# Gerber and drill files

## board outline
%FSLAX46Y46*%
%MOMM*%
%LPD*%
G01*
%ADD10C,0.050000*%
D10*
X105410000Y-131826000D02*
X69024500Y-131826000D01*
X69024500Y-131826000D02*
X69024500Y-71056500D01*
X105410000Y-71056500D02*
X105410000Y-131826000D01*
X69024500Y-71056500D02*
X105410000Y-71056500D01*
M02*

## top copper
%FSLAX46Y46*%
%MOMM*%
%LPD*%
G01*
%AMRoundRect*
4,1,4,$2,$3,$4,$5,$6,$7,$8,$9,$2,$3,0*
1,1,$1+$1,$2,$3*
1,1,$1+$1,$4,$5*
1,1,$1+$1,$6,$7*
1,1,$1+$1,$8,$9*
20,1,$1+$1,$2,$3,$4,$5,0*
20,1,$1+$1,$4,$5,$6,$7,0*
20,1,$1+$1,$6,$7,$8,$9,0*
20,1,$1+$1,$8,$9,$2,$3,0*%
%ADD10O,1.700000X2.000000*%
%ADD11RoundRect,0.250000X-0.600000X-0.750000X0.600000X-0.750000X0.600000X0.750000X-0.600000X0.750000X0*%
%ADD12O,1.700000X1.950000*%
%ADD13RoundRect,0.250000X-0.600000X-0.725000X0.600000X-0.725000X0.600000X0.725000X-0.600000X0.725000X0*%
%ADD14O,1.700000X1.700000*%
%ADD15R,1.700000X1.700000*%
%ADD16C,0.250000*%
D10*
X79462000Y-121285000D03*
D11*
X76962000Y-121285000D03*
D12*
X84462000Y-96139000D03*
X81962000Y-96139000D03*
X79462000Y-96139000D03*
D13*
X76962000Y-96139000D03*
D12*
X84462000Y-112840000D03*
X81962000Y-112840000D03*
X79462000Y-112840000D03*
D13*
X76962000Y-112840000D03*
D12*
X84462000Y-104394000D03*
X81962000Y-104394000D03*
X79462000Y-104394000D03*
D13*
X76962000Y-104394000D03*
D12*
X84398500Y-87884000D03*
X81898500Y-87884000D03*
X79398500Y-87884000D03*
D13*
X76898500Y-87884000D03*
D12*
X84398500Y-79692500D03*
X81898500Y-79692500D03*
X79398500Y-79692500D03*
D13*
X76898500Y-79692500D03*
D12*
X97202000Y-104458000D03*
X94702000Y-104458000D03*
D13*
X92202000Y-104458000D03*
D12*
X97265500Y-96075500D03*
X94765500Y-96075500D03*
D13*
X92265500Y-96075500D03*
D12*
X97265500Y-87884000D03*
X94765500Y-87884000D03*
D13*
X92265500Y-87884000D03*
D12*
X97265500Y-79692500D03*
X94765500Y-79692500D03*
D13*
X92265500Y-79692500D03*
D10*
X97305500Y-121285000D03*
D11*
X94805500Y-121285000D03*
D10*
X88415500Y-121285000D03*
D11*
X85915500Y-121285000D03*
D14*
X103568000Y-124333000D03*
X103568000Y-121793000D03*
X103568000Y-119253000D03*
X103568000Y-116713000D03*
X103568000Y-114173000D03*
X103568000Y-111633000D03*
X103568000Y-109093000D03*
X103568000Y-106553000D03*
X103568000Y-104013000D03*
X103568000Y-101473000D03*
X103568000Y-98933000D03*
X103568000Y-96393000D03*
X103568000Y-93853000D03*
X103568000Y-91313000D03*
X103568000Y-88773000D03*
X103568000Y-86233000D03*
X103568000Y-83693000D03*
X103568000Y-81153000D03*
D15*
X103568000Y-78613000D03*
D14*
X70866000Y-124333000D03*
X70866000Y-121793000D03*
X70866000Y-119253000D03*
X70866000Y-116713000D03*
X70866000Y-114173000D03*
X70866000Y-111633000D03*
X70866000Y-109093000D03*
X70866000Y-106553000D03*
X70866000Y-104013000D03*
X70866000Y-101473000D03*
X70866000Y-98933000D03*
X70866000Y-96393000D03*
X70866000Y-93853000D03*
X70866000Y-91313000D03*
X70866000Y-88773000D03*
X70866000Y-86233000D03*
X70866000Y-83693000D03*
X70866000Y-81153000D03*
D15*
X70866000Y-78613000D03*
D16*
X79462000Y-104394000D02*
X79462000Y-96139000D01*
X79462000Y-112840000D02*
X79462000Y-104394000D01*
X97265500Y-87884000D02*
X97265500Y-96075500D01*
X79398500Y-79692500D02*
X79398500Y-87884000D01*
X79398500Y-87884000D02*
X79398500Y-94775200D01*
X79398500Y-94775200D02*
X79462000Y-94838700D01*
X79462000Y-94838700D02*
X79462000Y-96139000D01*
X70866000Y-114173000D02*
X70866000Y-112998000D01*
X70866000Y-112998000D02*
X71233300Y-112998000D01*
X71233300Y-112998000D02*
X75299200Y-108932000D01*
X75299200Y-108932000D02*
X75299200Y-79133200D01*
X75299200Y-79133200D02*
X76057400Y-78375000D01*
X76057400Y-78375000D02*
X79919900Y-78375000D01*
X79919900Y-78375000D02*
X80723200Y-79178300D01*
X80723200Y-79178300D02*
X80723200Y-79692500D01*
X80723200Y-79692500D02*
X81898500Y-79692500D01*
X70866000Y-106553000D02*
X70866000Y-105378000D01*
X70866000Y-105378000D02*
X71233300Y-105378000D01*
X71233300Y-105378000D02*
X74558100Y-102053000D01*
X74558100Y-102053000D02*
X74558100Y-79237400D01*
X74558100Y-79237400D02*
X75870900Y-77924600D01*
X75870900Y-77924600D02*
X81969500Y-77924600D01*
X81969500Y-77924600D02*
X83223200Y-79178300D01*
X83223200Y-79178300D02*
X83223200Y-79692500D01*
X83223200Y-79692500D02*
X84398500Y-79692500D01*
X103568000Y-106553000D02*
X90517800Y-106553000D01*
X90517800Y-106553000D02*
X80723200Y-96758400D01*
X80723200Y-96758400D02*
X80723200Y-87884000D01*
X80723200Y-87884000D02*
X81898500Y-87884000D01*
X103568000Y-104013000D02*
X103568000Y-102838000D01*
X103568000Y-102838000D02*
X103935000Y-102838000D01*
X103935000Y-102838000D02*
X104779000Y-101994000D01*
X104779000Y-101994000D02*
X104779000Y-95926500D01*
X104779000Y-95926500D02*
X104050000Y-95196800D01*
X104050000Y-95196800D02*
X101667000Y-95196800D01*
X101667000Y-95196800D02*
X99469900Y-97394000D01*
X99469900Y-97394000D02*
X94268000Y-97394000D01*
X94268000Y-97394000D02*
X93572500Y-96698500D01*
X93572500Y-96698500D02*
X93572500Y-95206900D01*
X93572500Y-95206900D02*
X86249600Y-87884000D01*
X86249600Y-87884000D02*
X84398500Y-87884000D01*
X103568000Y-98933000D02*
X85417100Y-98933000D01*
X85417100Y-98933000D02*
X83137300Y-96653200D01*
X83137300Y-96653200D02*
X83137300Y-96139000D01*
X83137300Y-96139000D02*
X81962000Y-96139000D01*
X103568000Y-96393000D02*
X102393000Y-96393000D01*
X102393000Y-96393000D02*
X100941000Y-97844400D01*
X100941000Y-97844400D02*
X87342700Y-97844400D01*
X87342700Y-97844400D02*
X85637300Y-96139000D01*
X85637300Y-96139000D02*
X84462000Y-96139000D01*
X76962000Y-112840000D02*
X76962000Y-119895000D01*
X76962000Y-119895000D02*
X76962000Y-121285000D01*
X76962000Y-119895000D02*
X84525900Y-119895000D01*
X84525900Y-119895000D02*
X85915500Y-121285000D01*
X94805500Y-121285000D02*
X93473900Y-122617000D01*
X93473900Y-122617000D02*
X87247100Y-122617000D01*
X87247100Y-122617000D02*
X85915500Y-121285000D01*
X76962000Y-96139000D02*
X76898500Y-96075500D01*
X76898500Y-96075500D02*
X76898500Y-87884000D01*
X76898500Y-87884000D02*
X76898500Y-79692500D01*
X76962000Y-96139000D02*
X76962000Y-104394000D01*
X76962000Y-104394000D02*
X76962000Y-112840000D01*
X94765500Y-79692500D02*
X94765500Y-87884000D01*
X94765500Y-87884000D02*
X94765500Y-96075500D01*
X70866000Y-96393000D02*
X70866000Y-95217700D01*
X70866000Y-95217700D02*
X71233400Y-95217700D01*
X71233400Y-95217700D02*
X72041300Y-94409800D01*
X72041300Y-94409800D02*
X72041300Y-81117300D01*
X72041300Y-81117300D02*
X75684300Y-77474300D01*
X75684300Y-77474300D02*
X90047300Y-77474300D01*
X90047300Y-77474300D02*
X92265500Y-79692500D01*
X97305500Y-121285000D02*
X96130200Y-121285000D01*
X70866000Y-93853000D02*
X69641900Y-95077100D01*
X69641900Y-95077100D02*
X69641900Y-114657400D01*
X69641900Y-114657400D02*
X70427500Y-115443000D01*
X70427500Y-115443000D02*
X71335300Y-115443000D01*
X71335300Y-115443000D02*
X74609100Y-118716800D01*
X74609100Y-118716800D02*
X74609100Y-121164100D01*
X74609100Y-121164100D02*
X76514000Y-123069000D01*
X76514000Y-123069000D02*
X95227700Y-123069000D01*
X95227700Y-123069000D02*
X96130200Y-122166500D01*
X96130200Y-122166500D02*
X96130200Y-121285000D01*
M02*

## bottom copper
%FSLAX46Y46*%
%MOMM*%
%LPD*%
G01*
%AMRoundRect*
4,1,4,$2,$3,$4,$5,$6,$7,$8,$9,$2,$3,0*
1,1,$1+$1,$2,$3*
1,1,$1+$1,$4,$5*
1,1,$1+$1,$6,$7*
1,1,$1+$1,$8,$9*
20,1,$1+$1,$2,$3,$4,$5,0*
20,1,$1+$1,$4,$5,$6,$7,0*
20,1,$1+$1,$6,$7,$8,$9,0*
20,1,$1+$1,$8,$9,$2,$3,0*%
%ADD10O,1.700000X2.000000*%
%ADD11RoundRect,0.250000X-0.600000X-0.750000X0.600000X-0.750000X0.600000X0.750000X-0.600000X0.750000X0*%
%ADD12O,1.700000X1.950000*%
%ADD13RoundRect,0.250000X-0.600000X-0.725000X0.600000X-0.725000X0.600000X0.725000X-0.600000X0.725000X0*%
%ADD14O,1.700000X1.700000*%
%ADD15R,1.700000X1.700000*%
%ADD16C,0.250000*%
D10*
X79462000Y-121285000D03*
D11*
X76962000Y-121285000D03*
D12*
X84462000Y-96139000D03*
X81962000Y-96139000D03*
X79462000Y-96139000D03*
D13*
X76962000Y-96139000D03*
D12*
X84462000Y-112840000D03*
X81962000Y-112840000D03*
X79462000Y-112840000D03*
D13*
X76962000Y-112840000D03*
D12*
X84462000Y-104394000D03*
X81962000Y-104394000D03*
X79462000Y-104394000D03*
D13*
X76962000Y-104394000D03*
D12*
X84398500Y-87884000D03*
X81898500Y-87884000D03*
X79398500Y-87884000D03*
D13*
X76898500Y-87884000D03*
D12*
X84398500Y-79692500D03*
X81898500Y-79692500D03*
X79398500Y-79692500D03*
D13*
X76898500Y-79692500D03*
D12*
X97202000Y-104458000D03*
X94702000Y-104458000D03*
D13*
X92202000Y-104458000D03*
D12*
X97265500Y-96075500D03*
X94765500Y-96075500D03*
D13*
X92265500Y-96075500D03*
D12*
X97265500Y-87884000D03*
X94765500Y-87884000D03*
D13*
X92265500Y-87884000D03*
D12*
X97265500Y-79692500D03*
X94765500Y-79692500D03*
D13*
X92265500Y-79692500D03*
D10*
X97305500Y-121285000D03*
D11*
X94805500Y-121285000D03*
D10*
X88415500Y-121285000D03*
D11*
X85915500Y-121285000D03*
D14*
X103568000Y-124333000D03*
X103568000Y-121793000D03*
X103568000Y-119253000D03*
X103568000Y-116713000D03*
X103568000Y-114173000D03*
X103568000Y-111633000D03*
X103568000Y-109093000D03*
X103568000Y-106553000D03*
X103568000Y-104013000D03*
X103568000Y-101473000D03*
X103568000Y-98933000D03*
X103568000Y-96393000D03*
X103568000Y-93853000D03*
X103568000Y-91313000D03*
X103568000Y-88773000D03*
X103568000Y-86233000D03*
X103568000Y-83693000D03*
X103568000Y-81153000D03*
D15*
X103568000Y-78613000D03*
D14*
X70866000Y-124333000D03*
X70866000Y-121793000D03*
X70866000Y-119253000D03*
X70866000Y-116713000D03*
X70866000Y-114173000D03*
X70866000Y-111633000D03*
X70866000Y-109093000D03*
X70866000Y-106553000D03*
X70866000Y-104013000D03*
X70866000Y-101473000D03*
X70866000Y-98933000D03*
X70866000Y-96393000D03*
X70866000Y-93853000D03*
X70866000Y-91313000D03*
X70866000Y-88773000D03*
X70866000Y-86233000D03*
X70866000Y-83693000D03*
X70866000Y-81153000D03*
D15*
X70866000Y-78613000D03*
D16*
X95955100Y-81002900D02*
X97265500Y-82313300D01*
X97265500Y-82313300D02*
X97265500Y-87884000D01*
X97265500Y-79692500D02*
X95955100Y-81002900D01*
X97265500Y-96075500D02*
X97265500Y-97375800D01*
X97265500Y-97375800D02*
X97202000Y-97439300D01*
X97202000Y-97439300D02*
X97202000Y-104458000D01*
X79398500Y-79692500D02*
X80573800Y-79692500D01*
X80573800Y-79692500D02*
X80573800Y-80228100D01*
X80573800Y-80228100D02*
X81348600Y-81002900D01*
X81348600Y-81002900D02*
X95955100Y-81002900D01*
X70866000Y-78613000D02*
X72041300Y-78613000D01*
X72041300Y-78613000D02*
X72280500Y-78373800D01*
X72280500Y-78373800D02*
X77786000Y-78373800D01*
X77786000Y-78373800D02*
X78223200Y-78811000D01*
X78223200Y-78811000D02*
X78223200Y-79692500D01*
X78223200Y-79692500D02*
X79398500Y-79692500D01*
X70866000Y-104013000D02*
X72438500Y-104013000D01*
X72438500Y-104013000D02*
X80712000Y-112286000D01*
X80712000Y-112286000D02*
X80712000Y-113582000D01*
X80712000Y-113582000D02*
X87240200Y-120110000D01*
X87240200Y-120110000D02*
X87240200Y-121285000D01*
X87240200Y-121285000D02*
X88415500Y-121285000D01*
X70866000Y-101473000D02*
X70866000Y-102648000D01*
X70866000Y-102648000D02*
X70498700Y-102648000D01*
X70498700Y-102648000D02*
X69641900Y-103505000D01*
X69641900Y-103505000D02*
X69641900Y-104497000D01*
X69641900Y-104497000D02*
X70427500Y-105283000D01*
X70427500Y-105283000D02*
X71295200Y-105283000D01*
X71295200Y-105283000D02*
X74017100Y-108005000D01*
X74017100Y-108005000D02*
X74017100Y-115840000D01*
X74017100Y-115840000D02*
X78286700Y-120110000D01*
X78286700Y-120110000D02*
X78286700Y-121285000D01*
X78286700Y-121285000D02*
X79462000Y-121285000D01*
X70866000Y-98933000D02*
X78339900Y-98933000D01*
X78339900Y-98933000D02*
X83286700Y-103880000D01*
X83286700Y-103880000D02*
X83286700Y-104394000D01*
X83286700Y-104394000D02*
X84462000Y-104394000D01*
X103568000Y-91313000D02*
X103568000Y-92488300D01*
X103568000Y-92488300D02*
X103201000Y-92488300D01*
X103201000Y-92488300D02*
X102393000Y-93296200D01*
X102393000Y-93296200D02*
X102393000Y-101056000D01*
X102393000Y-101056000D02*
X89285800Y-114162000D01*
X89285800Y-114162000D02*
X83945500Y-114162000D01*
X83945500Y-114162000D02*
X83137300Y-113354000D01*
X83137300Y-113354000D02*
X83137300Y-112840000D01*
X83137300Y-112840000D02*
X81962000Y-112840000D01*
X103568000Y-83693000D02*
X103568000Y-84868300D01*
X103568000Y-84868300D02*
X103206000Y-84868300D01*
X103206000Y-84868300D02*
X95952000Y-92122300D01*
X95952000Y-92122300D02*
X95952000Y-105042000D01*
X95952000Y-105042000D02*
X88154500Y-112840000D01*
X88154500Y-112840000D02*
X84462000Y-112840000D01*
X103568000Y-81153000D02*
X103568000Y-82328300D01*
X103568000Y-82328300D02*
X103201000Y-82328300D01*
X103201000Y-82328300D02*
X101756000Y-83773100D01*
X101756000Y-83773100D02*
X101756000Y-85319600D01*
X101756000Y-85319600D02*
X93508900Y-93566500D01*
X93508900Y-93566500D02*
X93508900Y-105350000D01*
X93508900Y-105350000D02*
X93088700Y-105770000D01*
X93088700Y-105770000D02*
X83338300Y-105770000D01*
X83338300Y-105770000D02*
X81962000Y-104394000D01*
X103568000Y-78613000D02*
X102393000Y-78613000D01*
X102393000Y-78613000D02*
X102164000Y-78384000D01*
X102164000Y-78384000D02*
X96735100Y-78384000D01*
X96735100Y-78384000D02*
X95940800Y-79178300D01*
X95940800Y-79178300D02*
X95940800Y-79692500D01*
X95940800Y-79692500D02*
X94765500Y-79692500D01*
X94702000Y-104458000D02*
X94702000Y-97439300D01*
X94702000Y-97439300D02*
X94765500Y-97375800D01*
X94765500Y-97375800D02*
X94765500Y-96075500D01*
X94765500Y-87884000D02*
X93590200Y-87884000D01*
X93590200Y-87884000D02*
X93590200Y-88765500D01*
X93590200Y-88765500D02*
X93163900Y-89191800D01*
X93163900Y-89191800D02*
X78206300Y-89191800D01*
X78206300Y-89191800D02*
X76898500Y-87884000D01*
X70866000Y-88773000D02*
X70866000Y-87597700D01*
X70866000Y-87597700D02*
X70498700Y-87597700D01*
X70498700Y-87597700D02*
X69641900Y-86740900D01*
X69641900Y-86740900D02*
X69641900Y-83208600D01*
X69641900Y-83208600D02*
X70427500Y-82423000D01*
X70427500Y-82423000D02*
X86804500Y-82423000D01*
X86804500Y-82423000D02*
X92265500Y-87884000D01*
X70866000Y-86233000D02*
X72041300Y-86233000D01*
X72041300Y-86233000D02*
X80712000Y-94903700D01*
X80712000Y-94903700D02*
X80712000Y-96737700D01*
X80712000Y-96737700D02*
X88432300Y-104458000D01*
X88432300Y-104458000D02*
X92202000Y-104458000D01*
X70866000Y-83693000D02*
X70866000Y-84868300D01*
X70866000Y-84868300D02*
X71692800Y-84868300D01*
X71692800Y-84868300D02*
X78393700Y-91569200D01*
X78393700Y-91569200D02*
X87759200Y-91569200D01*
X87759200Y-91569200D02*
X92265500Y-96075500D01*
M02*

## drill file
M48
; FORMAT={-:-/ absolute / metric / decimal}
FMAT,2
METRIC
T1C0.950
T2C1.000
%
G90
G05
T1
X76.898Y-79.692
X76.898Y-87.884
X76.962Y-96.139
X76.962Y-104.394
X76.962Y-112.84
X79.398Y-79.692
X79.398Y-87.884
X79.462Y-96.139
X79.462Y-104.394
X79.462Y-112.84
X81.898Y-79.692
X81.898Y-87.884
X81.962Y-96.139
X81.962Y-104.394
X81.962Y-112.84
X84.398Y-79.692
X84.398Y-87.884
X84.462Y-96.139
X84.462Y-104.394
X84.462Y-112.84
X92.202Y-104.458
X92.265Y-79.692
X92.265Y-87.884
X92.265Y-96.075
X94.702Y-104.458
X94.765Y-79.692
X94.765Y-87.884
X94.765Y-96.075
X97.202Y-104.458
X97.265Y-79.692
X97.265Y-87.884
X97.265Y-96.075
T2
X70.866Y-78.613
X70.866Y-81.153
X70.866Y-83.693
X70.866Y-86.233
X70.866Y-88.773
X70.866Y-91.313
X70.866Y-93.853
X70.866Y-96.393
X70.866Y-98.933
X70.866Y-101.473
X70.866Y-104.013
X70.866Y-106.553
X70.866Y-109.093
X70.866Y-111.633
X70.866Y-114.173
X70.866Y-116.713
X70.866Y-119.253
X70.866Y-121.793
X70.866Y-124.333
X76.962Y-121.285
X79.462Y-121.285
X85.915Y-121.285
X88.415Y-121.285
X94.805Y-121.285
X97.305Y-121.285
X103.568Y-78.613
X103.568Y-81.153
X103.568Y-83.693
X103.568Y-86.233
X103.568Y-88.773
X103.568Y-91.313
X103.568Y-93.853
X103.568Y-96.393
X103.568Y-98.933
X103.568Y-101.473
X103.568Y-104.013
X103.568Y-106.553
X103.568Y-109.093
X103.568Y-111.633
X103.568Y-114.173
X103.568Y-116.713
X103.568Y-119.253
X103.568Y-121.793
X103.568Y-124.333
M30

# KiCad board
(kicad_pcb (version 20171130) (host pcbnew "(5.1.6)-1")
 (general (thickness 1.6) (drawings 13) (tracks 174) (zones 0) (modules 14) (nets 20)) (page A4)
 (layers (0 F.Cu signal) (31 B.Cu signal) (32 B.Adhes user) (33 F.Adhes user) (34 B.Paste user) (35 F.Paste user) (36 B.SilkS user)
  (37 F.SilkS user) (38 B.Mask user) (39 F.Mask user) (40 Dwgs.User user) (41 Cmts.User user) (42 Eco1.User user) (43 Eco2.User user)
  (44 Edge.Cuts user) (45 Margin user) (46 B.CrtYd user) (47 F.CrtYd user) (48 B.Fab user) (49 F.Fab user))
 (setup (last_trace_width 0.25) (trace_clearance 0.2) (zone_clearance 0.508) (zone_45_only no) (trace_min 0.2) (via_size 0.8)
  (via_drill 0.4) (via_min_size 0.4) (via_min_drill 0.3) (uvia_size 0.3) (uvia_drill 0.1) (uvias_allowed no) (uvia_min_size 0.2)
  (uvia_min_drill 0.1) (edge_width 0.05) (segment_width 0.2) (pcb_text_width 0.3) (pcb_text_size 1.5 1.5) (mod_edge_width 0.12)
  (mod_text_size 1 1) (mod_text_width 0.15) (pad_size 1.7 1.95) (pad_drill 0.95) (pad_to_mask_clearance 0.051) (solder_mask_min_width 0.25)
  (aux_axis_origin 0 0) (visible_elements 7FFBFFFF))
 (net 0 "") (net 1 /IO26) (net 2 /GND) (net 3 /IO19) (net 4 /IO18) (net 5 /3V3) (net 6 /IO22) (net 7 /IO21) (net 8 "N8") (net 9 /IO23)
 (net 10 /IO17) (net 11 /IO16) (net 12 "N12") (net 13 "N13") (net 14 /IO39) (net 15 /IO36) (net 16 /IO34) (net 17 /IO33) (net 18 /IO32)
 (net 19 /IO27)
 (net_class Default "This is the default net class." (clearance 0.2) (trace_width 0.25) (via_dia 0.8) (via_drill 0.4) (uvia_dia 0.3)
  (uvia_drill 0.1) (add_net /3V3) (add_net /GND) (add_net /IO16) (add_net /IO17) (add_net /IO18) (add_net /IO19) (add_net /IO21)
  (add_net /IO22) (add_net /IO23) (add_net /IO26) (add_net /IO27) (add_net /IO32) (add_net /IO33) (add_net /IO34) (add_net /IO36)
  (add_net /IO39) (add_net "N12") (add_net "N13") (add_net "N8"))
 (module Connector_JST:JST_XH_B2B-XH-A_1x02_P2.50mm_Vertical (layer F.Cu) (at 76.962 121.285)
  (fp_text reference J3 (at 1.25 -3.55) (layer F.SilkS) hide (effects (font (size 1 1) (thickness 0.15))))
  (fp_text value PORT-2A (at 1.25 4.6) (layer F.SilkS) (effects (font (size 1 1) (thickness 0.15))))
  (pad 2 thru_hole oval (at 2.5 0) (size 1.7 2) (drill 1) (layers *.Cu *.Mask) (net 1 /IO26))
  (pad 1 thru_hole roundrect (at 0 0) (size 1.7 2) (drill 1) (layers *.Cu *.Mask) (roundrect_rratio 0.147059) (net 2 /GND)))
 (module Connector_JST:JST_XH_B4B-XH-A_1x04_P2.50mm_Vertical (layer F.Cu) (at 76.962 96.139)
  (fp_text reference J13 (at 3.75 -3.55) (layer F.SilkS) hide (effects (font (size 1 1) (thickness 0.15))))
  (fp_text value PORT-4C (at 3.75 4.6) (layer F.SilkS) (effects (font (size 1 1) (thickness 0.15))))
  (pad 4 thru_hole oval (at 7.5 0) (size 1.7 1.95) (drill 0.95) (layers *.Cu *.Mask) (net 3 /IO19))
  (pad 3 thru_hole oval (at 5 0) (size 1.7 1.95) (drill 0.95) (layers *.Cu *.Mask) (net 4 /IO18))
  (pad 2 thru_hole oval (at 2.5 0) (size 1.7 1.95) (drill 0.95) (layers *.Cu *.Mask) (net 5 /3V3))
  (pad 1 thru_hole roundrect (at 0 0) (size 1.7 1.95) (drill 0.95) (layers *.Cu *.Mask) (roundrect_rratio 0.147059) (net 2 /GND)))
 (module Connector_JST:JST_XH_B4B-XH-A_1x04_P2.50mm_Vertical (layer F.Cu) (at 76.962 112.84)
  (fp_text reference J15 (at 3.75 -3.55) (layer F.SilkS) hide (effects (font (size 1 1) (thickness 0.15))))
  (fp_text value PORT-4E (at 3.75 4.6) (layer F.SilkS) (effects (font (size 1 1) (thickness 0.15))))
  (pad 4 thru_hole oval (at 7.5 0) (size 1.7 1.95) (drill 0.95) (layers *.Cu *.Mask) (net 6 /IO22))
  (pad 3 thru_hole oval (at 5 0) (size 1.7 1.95) (drill 0.95) (layers *.Cu *.Mask) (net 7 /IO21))
  (pad 2 thru_hole oval (at 2.5 0) (size 1.7 1.95) (drill 0.95) (layers *.Cu *.Mask) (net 5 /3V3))
  (pad 1 thru_hole roundrect (at 0 0) (size 1.7 1.95) (drill 0.95) (layers *.Cu *.Mask) (roundrect_rratio 0.147059) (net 2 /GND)))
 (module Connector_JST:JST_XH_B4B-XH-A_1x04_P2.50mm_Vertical (layer F.Cu) (at 76.962 104.394)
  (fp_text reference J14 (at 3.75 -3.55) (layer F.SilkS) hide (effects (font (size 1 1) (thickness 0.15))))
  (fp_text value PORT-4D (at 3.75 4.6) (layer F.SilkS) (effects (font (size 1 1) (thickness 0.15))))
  (pad 4 thru_hole oval (at 7.5 0) (size 1.7 1.95) (drill 0.95) (layers *.Cu *.Mask) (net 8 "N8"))
  (pad 3 thru_hole oval (at 5 0) (size 1.7 1.95) (drill 0.95) (layers *.Cu *.Mask) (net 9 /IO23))
  (pad 2 thru_hole oval (at 2.5 0) (size 1.7 1.95) (drill 0.95) (layers *.Cu *.Mask) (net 5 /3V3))
  (pad 1 thru_hole roundrect (at 0 0) (size 1.7 1.95) (drill 0.95) (layers *.Cu *.Mask) (roundrect_rratio 0.147059) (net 2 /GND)))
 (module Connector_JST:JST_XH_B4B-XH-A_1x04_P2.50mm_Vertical (layer F.Cu) (at 76.8985 87.884)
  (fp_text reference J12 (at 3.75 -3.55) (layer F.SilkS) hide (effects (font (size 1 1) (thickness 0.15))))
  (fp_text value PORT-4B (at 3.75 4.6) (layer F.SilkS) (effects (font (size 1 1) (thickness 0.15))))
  (pad 4 thru_hole oval (at 7.5 0) (size 1.7 1.95) (drill 0.95) (layers *.Cu *.Mask) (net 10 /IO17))
  (pad 3 thru_hole oval (at 5 0) (size 1.7 1.95) (drill 0.95) (layers *.Cu *.Mask) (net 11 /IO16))
  (pad 2 thru_hole oval (at 2.5 0) (size 1.7 1.95) (drill 0.95) (layers *.Cu *.Mask) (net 5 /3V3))
  (pad 1 thru_hole roundrect (at 0 0) (size 1.7 1.95) (drill 0.95) (layers *.Cu *.Mask) (roundrect_rratio 0.147059) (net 2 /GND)))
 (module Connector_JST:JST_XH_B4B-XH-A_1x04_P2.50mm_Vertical (layer F.Cu) (at 76.8985 79.6925)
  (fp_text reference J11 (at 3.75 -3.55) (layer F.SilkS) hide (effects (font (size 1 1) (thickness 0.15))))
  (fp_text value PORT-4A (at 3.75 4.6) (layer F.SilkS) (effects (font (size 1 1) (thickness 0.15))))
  (pad 4 thru_hole oval (at 7.5 0) (size 1.7 1.95) (drill 0.95) (layers *.Cu *.Mask) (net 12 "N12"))
  (pad 3 thru_hole oval (at 5 0) (size 1.7 1.95) (drill 0.95) (layers *.Cu *.Mask) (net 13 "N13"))
  (pad 2 thru_hole oval (at 2.5 0) (size 1.7 1.95) (drill 0.95) (layers *.Cu *.Mask) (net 5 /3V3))
  (pad 1 thru_hole roundrect (at 0 0) (size 1.7 1.95) (drill 0.95) (layers *.Cu *.Mask) (roundrect_rratio 0.147059) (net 2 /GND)))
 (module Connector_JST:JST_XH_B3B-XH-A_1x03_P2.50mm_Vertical (layer F.Cu) (at 92.202 104.458)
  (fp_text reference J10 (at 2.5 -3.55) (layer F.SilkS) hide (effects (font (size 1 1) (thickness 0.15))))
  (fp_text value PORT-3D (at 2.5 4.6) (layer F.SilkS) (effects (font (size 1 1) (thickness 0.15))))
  (pad 3 thru_hole oval (at 5 0) (size 1.7 1.95) (drill 0.95) (layers *.Cu *.Mask) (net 5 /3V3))
  (pad 2 thru_hole oval (at 2.5 0) (size 1.7 1.95) (drill 0.95) (layers *.Cu *.Mask) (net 2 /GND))
  (pad 1 thru_hole roundrect (at 0 0) (size 1.7 1.95) (drill 0.95) (layers *.Cu *.Mask) (roundrect_rratio 0.147059) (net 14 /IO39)))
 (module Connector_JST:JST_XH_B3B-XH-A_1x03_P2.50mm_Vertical (layer F.Cu) (at 92.2655 96.0755)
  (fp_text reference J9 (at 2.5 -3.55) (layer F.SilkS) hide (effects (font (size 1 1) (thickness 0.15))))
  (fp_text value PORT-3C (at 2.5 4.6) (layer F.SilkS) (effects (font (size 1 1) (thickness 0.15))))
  (pad 3 thru_hole oval (at 5 0) (size 1.7 1.95) (drill 0.95) (layers *.Cu *.Mask) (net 5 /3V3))
  (pad 2 thru_hole oval (at 2.5 0) (size 1.7 1.95) (drill 0.95) (layers *.Cu *.Mask) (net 2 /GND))
  (pad 1 thru_hole roundrect (at 0 0) (size 1.7 1.95) (drill 0.95) (layers *.Cu *.Mask) (roundrect_rratio 0.147059) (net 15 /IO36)))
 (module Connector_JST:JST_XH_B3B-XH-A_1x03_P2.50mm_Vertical (layer F.Cu) (at 92.2655 87.884)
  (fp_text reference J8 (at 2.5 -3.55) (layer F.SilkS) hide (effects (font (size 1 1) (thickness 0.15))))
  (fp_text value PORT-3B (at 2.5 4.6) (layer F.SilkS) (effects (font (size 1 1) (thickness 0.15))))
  (pad 3 thru_hole oval (at 5 0) (size 1.7 1.95) (drill 0.95) (layers *.Cu *.Mask) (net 5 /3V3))
  (pad 2 thru_hole oval (at 2.5 0) (size 1.7 1.95) (drill 0.95) (layers *.Cu *.Mask) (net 2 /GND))
  (pad 1 thru_hole roundrect (at 0 0) (size 1.7 1.95) (drill 0.95) (layers *.Cu *.Mask) (roundrect_rratio 0.147059) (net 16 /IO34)))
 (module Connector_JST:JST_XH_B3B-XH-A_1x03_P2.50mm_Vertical (layer F.Cu) (at 92.2655 79.6925)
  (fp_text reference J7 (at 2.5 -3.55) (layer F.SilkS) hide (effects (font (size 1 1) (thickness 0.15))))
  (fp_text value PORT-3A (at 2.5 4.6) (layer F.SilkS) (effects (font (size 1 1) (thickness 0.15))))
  (pad 3 thru_hole oval (at 5 0) (size 1.7 1.95) (drill 0.95) (layers *.Cu *.Mask) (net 5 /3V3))
  (pad 2 thru_hole oval (at 2.5 0) (size 1.7 1.95) (drill 0.95) (layers *.Cu *.Mask) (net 2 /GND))
  (pad 1 thru_hole roundrect (at 0 0) (size 1.7 1.95) (drill 0.95) (layers *.Cu *.Mask) (roundrect_rratio 0.147059) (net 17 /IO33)))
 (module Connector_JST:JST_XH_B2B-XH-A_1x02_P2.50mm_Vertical (layer F.Cu) (at 94.8055 121.285)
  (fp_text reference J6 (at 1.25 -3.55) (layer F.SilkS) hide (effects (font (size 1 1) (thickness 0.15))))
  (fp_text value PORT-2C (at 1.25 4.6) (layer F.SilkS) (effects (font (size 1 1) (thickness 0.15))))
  (pad 2 thru_hole oval (at 2.5 0) (size 1.7 2) (drill 1) (layers *.Cu *.Mask) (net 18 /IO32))
  (pad 1 thru_hole roundrect (at 0 0) (size 1.7 2) (drill 1) (layers *.Cu *.Mask) (roundrect_rratio 0.147059) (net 2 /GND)))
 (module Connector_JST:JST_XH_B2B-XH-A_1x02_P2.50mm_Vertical (layer F.Cu) (at 85.9155 121.285)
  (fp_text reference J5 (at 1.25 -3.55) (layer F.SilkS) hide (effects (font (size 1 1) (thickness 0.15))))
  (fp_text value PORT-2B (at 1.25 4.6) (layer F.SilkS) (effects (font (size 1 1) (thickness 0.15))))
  (pad 2 thru_hole oval (at 2.5 0) (size 1.7 2) (drill 1) (layers *.Cu *.Mask) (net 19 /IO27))
  (pad 1 thru_hole roundrect (at 0 0) (size 1.7 2) (drill 1) (layers *.Cu *.Mask) (roundrect_rratio 0.147059) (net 2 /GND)))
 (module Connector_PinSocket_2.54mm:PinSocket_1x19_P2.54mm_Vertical (layer F.Cu) (at 103.568 78.613)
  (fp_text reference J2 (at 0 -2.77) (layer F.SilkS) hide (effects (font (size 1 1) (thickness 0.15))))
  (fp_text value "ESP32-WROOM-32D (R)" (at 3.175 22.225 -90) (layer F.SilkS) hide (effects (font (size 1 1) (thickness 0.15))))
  (pad 19 thru_hole oval (at 0 45.72) (size 1.7 1.7) (drill 1) (layers *.Cu *.Mask))
  (pad 18 thru_hole oval (at 0 43.18) (size 1.7 1.7) (drill 1) (layers *.Cu *.Mask))
  (pad 17 thru_hole oval (at 0 40.64) (size 1.7 1.7) (drill 1) (layers *.Cu *.Mask))
  (pad 16 thru_hole oval (at 0 38.1) (size 1.7 1.7) (drill 1) (layers *.Cu *.Mask))
  (pad 15 thru_hole oval (at 0 35.56) (size 1.7 1.7) (drill 1) (layers *.Cu *.Mask))
  (pad 14 thru_hole oval (at 0 33.02) (size 1.7 1.7) (drill 1) (layers *.Cu *.Mask))
  (pad 13 thru_hole oval (at 0 30.48) (size 1.7 1.7) (drill 1) (layers *.Cu *.Mask))
  (pad 12 thru_hole oval (at 0 27.94) (size 1.7 1.7) (drill 1) (layers *.Cu *.Mask) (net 11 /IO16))
  (pad 11 thru_hole oval (at 0 25.4) (size 1.7 1.7) (drill 1) (layers *.Cu *.Mask) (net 10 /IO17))
  (pad 10 thru_hole oval (at 0 22.86) (size 1.7 1.7) (drill 1) (layers *.Cu *.Mask))
  (pad 9 thru_hole oval (at 0 20.32) (size 1.7 1.7) (drill 1) (layers *.Cu *.Mask) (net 4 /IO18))
  (pad 8 thru_hole oval (at 0 17.78) (size 1.7 1.7) (drill 1) (layers *.Cu *.Mask) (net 3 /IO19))
  (pad 7 thru_hole oval (at 0 15.24) (size 1.7 1.7) (drill 1) (layers *.Cu *.Mask))
  (pad 6 thru_hole oval (at 0 12.7) (size 1.7 1.7) (drill 1) (layers *.Cu *.Mask) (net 7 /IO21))
  (pad 5 thru_hole oval (at 0 10.16) (size 1.7 1.7) (drill 1) (layers *.Cu *.Mask))
  (pad 4 thru_hole oval (at 0 7.62) (size 1.7 1.7) (drill 1) (layers *.Cu *.Mask))
  (pad 3 thru_hole oval (at 0 5.08) (size 1.7 1.7) (drill 1) (layers *.Cu *.Mask) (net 6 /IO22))
  (pad 2 thru_hole oval (at 0 2.54) (size 1.7 1.7) (drill 1) (layers *.Cu *.Mask) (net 9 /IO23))
  (pad 1 thru_hole rect (at 0 0) (size 1.7 1.7) (drill 1) (layers *.Cu *.Mask) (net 2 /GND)))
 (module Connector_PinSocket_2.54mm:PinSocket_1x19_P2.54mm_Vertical (layer F.Cu) (at 70.866 78.613)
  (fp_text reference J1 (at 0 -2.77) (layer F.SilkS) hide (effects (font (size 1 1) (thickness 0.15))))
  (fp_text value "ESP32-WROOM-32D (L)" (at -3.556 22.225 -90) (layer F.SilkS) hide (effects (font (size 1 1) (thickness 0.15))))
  (pad 19 thru_hole oval (at 0 45.72) (size 1.7 1.7) (drill 1) (layers *.Cu *.Mask))
  (pad 18 thru_hole oval (at 0 43.18) (size 1.7 1.7) (drill 1) (layers *.Cu *.Mask))
  (pad 17 thru_hole oval (at 0 40.64) (size 1.7 1.7) (drill 1) (layers *.Cu *.Mask))
  (pad 16 thru_hole oval (at 0 38.1) (size 1.7 1.7) (drill 1) (layers *.Cu *.Mask))
  (pad 15 thru_hole oval (at 0 35.56) (size 1.7 1.7) (drill 1) (layers *.Cu *.Mask) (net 13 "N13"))
  (pad 14 thru_hole oval (at 0 33.02) (size 1.7 1.7) (drill 1) (layers *.Cu *.Mask))
  (pad 13 thru_hole oval (at 0 30.48) (size 1.7 1.7) (drill 1) (layers *.Cu *.Mask))
  (pad 12 thru_hole oval (at 0 27.94) (size 1.7 1.7) (drill 1) (layers *.Cu *.Mask) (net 12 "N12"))
  (pad 11 thru_hole oval (at 0 25.4) (size 1.7 1.7) (drill 1) (layers *.Cu *.Mask) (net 19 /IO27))
  (pad 10 thru_hole oval (at 0 22.86) (size 1.7 1.7) (drill 1) (layers *.Cu *.Mask) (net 1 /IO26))
  (pad 9 thru_hole oval (at 0 20.32) (size 1.7 1.7) (drill 1) (layers *.Cu *.Mask) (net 8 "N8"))
  (pad 8 thru_hole oval (at 0 17.78) (size 1.7 1.7) (drill 1) (layers *.Cu *.Mask) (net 17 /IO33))
  (pad 7 thru_hole oval (at 0 15.24) (size 1.7 1.7) (drill 1) (layers *.Cu *.Mask) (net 18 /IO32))
  (pad 6 thru_hole oval (at 0 12.7) (size 1.7 1.7) (drill 1) (layers *.Cu *.Mask))
  (pad 5 thru_hole oval (at 0 10.16) (size 1.7 1.7) (drill 1) (layers *.Cu *.Mask) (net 16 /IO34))
  (pad 4 thru_hole oval (at 0 7.62) (size 1.7 1.7) (drill 1) (layers *.Cu *.Mask) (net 14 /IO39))
  (pad 3 thru_hole oval (at 0 5.08) (size 1.7 1.7) (drill 1) (layers *.Cu *.Mask) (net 15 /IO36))
  (pad 2 thru_hole oval (at 0 2.54) (size 1.7 1.7) (drill 1) (layers *.Cu *.Mask))
  (pad 1 thru_hole rect (at 0 0) (size 1.7 1.7) (drill 1) (layers *.Cu *.Mask) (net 5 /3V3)))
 (gr_line (start 105.41 131.826) (end 69.0245 131.826) (layer Edge.Cuts) (width 0.05))
 (gr_line (start 69.0245 131.826) (end 69.0245 71.0565) (layer Edge.Cuts) (width 0.05))
 (gr_line (start 105.41 71.0565) (end 105.41 131.826) (layer Edge.Cuts) (width 0.05))
 (gr_line (start 69.0245 71.0565) (end 105.41 71.0565) (layer Edge.Cuts) (width 0.05))
 (segment (start 95.9551 81.0029) (end 97.2655 82.3133) (width 0.25) (layer B.Cu) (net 5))
 (segment (start 97.2655 82.3133) (end 97.2655 87.884) (width 0.25) (layer B.Cu) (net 5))
 (segment (start 97.2655 79.6925) (end 95.9551 81.0029) (width 0.25) (layer B.Cu) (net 5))
 (segment (start 79.462 104.394) (end 79.462 96.139) (width 0.25) (layer F.Cu) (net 5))
 (segment (start 79.462 112.84) (end 79.462 104.394) (width 0.25) (layer F.Cu) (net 5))
 (segment (start 97.2655 87.884) (end 97.2655 96.0755) (width 0.25) (layer F.Cu) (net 5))
 (segment (start 97.2655 96.0755) (end 97.2655 97.3758) (width 0.25) (layer B.Cu) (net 5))
 (segment (start 97.2655 97.3758) (end 97.202 97.4393) (width 0.25) (layer B.Cu) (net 5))
 (segment (start 97.202 97.4393) (end 97.202 104.458) (width 0.25) (layer B.Cu) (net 5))
 (segment (start 79.3985 79.6925) (end 80.5738 79.6925) (width 0.25) (layer B.Cu) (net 5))
 (segment (start 80.5738 79.6925) (end 80.5738 80.2281) (width 0.25) (layer B.Cu) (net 5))
 (segment (start 80.5738 80.2281) (end 81.3486 81.0029) (width 0.25) (layer B.Cu) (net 5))
 (segment (start 81.3486 81.0029) (end 95.9551 81.0029) (width 0.25) (layer B.Cu) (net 5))
 (segment (start 79.3985 79.6925) (end 79.3985 87.884) (width 0.25) (layer F.Cu) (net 5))
 (segment (start 79.3985 87.884) (end 79.3985 94.7752) (width 0.25) (layer F.Cu) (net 5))
 (segment (start 79.3985 94.7752) (end 79.462 94.8387) (width 0.25) (layer F.Cu) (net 5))
 (segment (start 79.462 94.8387) (end 79.462 96.139) (width 0.25) (layer F.Cu) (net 5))
 (segment (start 70.866 78.613) (end 72.0413 78.613) (width 0.25) (layer B.Cu) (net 5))
 (segment (start 72.0413 78.613) (end 72.2805 78.3738) (width 0.25) (layer B.Cu) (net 5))
 (segment (start 72.2805 78.3738) (end 77.786 78.3738) (width 0.25) (layer B.Cu) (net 5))
 (segment (start 77.786 78.3738) (end 78.2232 78.811) (width 0.25) (layer B.Cu) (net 5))
 (segment (start 78.2232 78.811) (end 78.2232 79.6925) (width 0.25) (layer B.Cu) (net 5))
 (segment (start 78.2232 79.6925) (end 79.3985 79.6925) (width 0.25) (layer B.Cu) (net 5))
 (segment (start 70.866 114.173) (end 70.866 112.998) (width 0.25) (layer F.Cu) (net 13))
 (segment (start 70.866 112.998) (end 71.2333 112.998) (width 0.25) (layer F.Cu) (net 13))
 (segment (start 71.2333 112.998) (end 75.2992 108.932) (width 0.25) (layer F.Cu) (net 13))
 (segment (start 75.2992 108.932) (end 75.2992 79.1332) (width 0.25) (layer F.Cu) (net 13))
 (segment (start 75.2992 79.1332) (end 76.0574 78.375) (width 0.25) (layer F.Cu) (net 13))
 (segment (start 76.0574 78.375) (end 79.9199 78.375) (width 0.25) (layer F.Cu) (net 13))
 (segment (start 79.9199 78.375) (end 80.7232 79.1783) (width 0.25) (layer F.Cu) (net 13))
 (segment (start 80.7232 79.1783) (end 80.7232 79.6925) (width 0.25) (layer F.Cu) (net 13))
 (segment (start 80.7232 79.6925) (end 81.8985 79.6925) (width 0.25) (layer F.Cu) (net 13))
 (segment (start 70.866 106.553) (end 70.866 105.378) (width 0.25) (layer F.Cu) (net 12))
 (segment (start 70.866 105.378) (end 71.2333 105.378) (width 0.25) (layer F.Cu) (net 12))
 (segment (start 71.2333 105.378) (end 74.5581 102.053) (width 0.25) (layer F.Cu) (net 12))
 (segment (start 74.5581 102.053) (end 74.5581 79.2374) (width 0.25) (layer F.Cu) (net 12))
 (segment (start 74.5581 79.2374) (end 75.8709 77.9246) (width 0.25) (layer F.Cu) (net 12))
 (segment (start 75.8709 77.9246) (end 81.9695 77.9246) (width 0.25) (layer F.Cu) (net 12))
 (segment (start 81.9695 77.9246) (end 83.2232 79.1783) (width 0.25) (layer F.Cu) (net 12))
 (segment (start 83.2232 79.1783) (end 83.2232 79.6925) (width 0.25) (layer F.Cu) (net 12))
 (segment (start 83.2232 79.6925) (end 84.3985 79.6925) (width 0.25) (layer F.Cu) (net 12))
 (segment (start 70.866 104.013) (end 72.4385 104.013) (width 0.25) (layer B.Cu) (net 19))
 (segment (start 72.4385 104.013) (end 80.712 112.286) (width 0.25) (layer B.Cu) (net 19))
 (segment (start 80.712 112.286) (end 80.712 113.582) (width 0.25) (layer B.Cu) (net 19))
 (segment (start 80.712 113.582) (end 87.2402 120.11) (width 0.25) (layer B.Cu) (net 19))
 (segment (start 87.2402 120.11) (end 87.2402 121.285) (width 0.25) (layer B.Cu) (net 19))
 (segment (start 87.2402 121.285) (end 88.4155 121.285) (width 0.25) (layer B.Cu) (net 19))
 (segment (start 70.866 101.473) (end 70.866 102.648) (width 0.25) (layer B.Cu) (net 1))
 (segment (start 70.866 102.648) (end 70.4987 102.648) (width 0.25) (layer B.Cu) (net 1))
 (segment (start 70.4987 102.648) (end 69.6419 103.505) (width 0.25) (layer B.Cu) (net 1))
 (segment (start 69.6419 103.505) (end 69.6419 104.497) (width 0.25) (layer B.Cu) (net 1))
 (segment (start 69.6419 104.497) (end 70.4275 105.283) (width 0.25) (layer B.Cu) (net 1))
 (segment (start 70.4275 105.283) (end 71.2952 105.283) (width 0.25) (layer B.Cu) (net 1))
 (segment (start 71.2952 105.283) (end 74.0171 108.005) (width 0.25) (layer B.Cu) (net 1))
 (segment (start 74.0171 108.005) (end 74.0171 115.84) (width 0.25) (layer B.Cu) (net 1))
 (segment (start 74.0171 115.84) (end 78.2867 120.11) (width 0.25) (layer B.Cu) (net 1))
 (segment (start 78.2867 120.11) (end 78.2867 121.285) (width 0.25) (layer B.Cu) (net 1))
 (segment (start 78.2867 121.285) (end 79.462 121.285) (width 0.25) (layer B.Cu) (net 1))
 (segment (start 70.866 98.933) (end 78.3399 98.933) (width 0.25) (layer B.Cu) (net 8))
 (segment (start 78.3399 98.933) (end 83.2867 103.88) (width 0.25) (layer B.Cu) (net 8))
 (segment (start 83.2867 103.88) (end 83.2867 104.394) (width 0.25) (layer B.Cu) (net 8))
 (segment (start 83.2867 104.394) (end 84.462 104.394) (width 0.25) (layer B.Cu) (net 8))
 (segment (start 103.568 106.553) (end 90.5178 106.553) (width 0.25) (layer F.Cu) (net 11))
 (segment (start 90.5178 106.553) (end 80.7232 96.7584) (width 0.25) (layer F.Cu) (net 11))
 (segment (start 80.7232 96.7584) (end 80.7232 87.884) (width 0.25) (layer F.Cu) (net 11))
 (segment (start 80.7232 87.884) (end 81.8985 87.884) (width 0.25) (layer F.Cu) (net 11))
 (segment (start 103.568 104.013) (end 103.568 102.838) (width 0.25) (layer F.Cu) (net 10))
 (segment (start 103.568 102.838) (end 103.935 102.838) (width 0.25) (layer F.Cu) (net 10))
 (segment (start 103.935 102.838) (end 104.779 101.994) (width 0.25) (layer F.Cu) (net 10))
 (segment (start 104.779 101.994) (end 104.779 95.9265) (width 0.25) (layer F.Cu) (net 10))
 (segment (start 104.779 95.9265) (end 104.05 95.1968) (width 0.25) (layer F.Cu) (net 10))
 (segment (start 104.05 95.1968) (end 101.667 95.1968) (width 0.25) (layer F.Cu) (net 10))
 (segment (start 101.667 95.1968) (end 99.4699 97.394) (width 0.25) (layer F.Cu) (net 10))
 (segment (start 99.4699 97.394) (end 94.268 97.394) (width 0.25) (layer F.Cu) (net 10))
 (segment (start 94.268 97.394) (end 93.5725 96.6985) (width 0.25) (layer F.Cu) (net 10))
 (segment (start 93.5725 96.6985) (end 93.5725 95.2069) (width 0.25) (layer F.Cu) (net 10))
 (segment (start 93.5725 95.2069) (end 86.2496 87.884) (width 0.25) (layer F.Cu) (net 10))
 (segment (start 86.2496 87.884) (end 84.3985 87.884) (width 0.25) (layer F.Cu) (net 10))
 (segment (start 103.568 98.933) (end 85.4171 98.933) (width 0.25) (layer F.Cu) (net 4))
 (segment (start 85.4171 98.933) (end 83.1373 96.6532) (width 0.25) (layer F.Cu) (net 4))
 (segment (start 83.1373 96.6532) (end 83.1373 96.139) (width 0.25) (layer F.Cu) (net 4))
 (segment (start 83.1373 96.139) (end 81.962 96.139) (width 0.25) (layer F.Cu) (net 4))
 (segment (start 103.568 96.393) (end 102.393 96.393) (width 0.25) (layer F.Cu) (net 3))
 (segment (start 102.393 96.393) (end 100.941 97.8444) (width 0.25) (layer F.Cu) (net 3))
 (segment (start 100.941 97.8444) (end 87.3427 97.8444) (width 0.25) (layer F.Cu) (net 3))
 (segment (start 87.3427 97.8444) (end 85.6373 96.139) (width 0.25) (layer F.Cu) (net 3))
 (segment (start 85.6373 96.139) (end 84.462 96.139) (width 0.25) (layer F.Cu) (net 3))
 (segment (start 103.568 91.313) (end 103.568 92.4883) (width 0.25) (layer B.Cu) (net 7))
 (segment (start 103.568 92.4883) (end 103.201 92.4883) (width 0.25) (layer B.Cu) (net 7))
 (segment (start 103.201 92.4883) (end 102.393 93.2962) (width 0.25) (layer B.Cu) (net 7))
 (segment (start 102.393 93.2962) (end 102.393 101.056) (width 0.25) (layer B.Cu) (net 7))
 (segment (start 102.393 101.056) (end 89.2858 114.162) (width 0.25) (layer B.Cu) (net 7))
 (segment (start 89.2858 114.162) (end 83.9455 114.162) (width 0.25) (layer B.Cu) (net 7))
 (segment (start 83.9455 114.162) (end 83.1373 113.354) (width 0.25) (layer B.Cu) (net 7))
 (segment (start 83.1373 113.354) (end 83.1373 112.84) (width 0.25) (layer B.Cu) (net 7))
 (segment (start 83.1373 112.84) (end 81.962 112.84) (width 0.25) (layer B.Cu) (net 7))
 (segment (start 103.568 83.693) (end 103.568 84.8683) (width 0.25) (layer B.Cu) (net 6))
 (segment (start 103.568 84.8683) (end 103.206 84.8683) (width 0.25) (layer B.Cu) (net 6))
 (segment (start 103.206 84.8683) (end 95.952 92.1223) (width 0.25) (layer B.Cu) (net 6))
 (segment (start 95.952 92.1223) (end 95.952 105.042) (width 0.25) (layer B.Cu) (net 6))
 (segment (start 95.952 105.042) (end 88.1545 112.84) (width 0.25) (layer B.Cu) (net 6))
 (segment (start 88.1545 112.84) (end 84.462 112.84) (width 0.25) (layer B.Cu) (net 6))
 (segment (start 103.568 81.153) (end 103.568 82.3283) (width 0.25) (layer B.Cu) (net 9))
 (segment (start 103.568 82.3283) (end 103.201 82.3283) (width 0.25) (layer B.Cu) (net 9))
 (segment (start 103.201 82.3283) (end 101.756 83.7731) (width 0.25) (layer B.Cu) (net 9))
 (segment (start 101.756 83.7731) (end 101.756 85.3196) (width 0.25) (layer B.Cu) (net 9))
 (segment (start 101.756 85.3196) (end 93.5089 93.5665) (width 0.25) (layer B.Cu) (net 9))
 (segment (start 93.5089 93.5665) (end 93.5089 105.35) (width 0.25) (layer B.Cu) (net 9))
 (segment (start 93.5089 105.35) (end 93.0887 105.77) (width 0.25) (layer B.Cu) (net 9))
 (segment (start 93.0887 105.77) (end 83.3383 105.77) (width 0.25) (layer B.Cu) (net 9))
 (segment (start 83.3383 105.77) (end 81.962 104.394) (width 0.25) (layer B.Cu) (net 9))
 (segment (start 103.568 78.613) (end 102.393 78.613) (width 0.25) (layer B.Cu) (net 2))
 (segment (start 102.393 78.613) (end 102.164 78.384) (width 0.25) (layer B.Cu) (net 2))
 (segment (start 102.164 78.384) (end 96.7351 78.384) (width 0.25) (layer B.Cu) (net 2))
 (segment (start 96.7351 78.384) (end 95.9408 79.1783) (width 0.25) (layer B.Cu) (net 2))
 (segment (start 95.9408 79.1783) (end 95.9408 79.6925) (width 0.25) (layer B.Cu) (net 2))
 (segment (start 95.9408 79.6925) (end 94.7655 79.6925) (width 0.25) (layer B.Cu) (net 2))
 (segment (start 76.962 112.84) (end 76.962 119.895) (width 0.25) (layer F.Cu) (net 2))
 (segment (start 76.962 119.895) (end 76.962 121.285) (width 0.25) (layer F.Cu) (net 2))
 (segment (start 76.962 119.895) (end 84.5259 119.895) (width 0.25) (layer F.Cu) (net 2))
 (segment (start 84.5259 119.895) (end 85.9155 121.285) (width 0.25) (layer F.Cu) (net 2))
 (segment (start 94.8055 121.285) (end 93.4739 122.617) (width 0.25) (layer F.Cu) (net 2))
 (segment (start 93.4739 122.617) (end 87.2471 122.617) (width 0.25) (layer F.Cu) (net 2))
 (segment (start 87.2471 122.617) (end 85.9155 121.285) (width 0.25) (layer F.Cu) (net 2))
 (segment (start 76.962 96.139) (end 76.8985 96.0755) (width 0.25) (layer F.Cu) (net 2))
 (segment (start 76.8985 96.0755) (end 76.8985 87.884) (width 0.25) (layer F.Cu) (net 2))
 (segment (start 76.8985 87.884) (end 76.8985 79.6925) (width 0.25) (layer F.Cu) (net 2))
 (segment (start 76.962 96.139) (end 76.962 104.394) (width 0.25) (layer F.Cu) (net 2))
 (segment (start 76.962 104.394) (end 76.962 112.84) (width 0.25) (layer F.Cu) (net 2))
 (segment (start 94.702 104.458) (end 94.702 97.4393) (width 0.25) (layer B.Cu) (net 2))
 (segment (start 94.702 97.4393) (end 94.7655 97.3758) (width 0.25) (layer B.Cu) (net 2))
 (segment (start 94.7655 97.3758) (end 94.7655 96.0755) (width 0.25) (layer B.Cu) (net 2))
 (segment (start 94.7655 79.6925) (end 94.7655 87.884) (width 0.25) (layer F.Cu) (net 2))
 (segment (start 94.7655 87.884) (end 94.7655 96.0755) (width 0.25) (layer F.Cu) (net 2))
 (segment (start 94.7655 87.884) (end 93.5902 87.884) (width 0.25) (layer B.Cu) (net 2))
 (segment (start 93.5902 87.884) (end 93.5902 88.7655) (width 0.25) (layer B.Cu) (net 2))
 (segment (start 93.5902 88.7655) (end 93.1639 89.1918) (width 0.25) (layer B.Cu) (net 2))
 (segment (start 93.1639 89.1918) (end 78.2063 89.1918) (width 0.25) (layer B.Cu) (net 2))
 (segment (start 78.2063 89.1918) (end 76.8985 87.884) (width 0.25) (layer B.Cu) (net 2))
 (segment (start 70.866 88.773) (end 70.866 87.5977) (width 0.25) (layer B.Cu) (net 16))
 (segment (start 70.866 87.5977) (end 70.4987 87.5977) (width 0.25) (layer B.Cu) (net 16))
 (segment (start 70.4987 87.5977) (end 69.6419 86.7409) (width 0.25) (layer B.Cu) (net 16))
 (segment (start 69.6419 86.7409) (end 69.6419 83.2086) (width 0.25) (layer B.Cu) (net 16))
 (segment (start 69.6419 83.2086) (end 70.4275 82.423) (width 0.25) (layer B.Cu) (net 16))
 (segment (start 70.4275 82.423) (end 86.8045 82.423) (width 0.25) (layer B.Cu) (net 16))
 (segment (start 86.8045 82.423) (end 92.2655 87.884) (width 0.25) (layer B.Cu) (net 16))
 (segment (start 70.866 86.233) (end 72.0413 86.233) (width 0.25) (layer B.Cu) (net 14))
 (segment (start 72.0413 86.233) (end 80.712 94.9037) (width 0.25) (layer B.Cu) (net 14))
 (segment (start 80.712 94.9037) (end 80.712 96.7377) (width 0.25) (layer B.Cu) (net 14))
 (segment (start 80.712 96.7377) (end 88.4323 104.458) (width 0.25) (layer B.Cu) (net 14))
 (segment (start 88.4323 104.458) (end 92.202 104.458) (width 0.25) (layer B.Cu) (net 14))
 (segment (start 70.866 83.693) (end 70.866 84.8683) (width 0.25) (layer B.Cu) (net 15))
 (segment (start 70.866 84.8683) (end 71.6928 84.8683) (width 0.25) (layer B.Cu) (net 15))
 (segment (start 71.6928 84.8683) (end 78.3937 91.5692) (width 0.25) (layer B.Cu) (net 15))
 (segment (start 78.3937 91.5692) (end 87.7592 91.5692) (width 0.25) (layer B.Cu) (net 15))
 (segment (start 87.7592 91.5692) (end 92.2655 96.0755) (width 0.25) (layer B.Cu) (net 15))
 (segment (start 70.866 96.393) (end 70.866 95.2177) (width 0.25) (layer F.Cu) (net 17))
 (segment (start 70.866 95.2177) (end 71.2334 95.2177) (width 0.25) (layer F.Cu) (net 17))
 (segment (start 71.2334 95.2177) (end 72.0413 94.4098) (width 0.25) (layer F.Cu) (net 17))
 (segment (start 72.0413 94.4098) (end 72.0413 81.1173) (width 0.25) (layer F.Cu) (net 17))
 (segment (start 72.0413 81.1173) (end 75.6843 77.4743) (width 0.25) (layer F.Cu) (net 17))
 (segment (start 75.6843 77.4743) (end 90.0473 77.4743) (width 0.25) (layer F.Cu) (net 17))
 (segment (start 90.0473 77.4743) (end 92.2655 79.6925) (width 0.25) (layer F.Cu) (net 17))
 (segment (start 97.3055 121.285) (end 96.1302 121.285) (width 0.25) (layer F.Cu) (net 18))
 (segment (start 70.866 93.853) (end 69.6419 95.0771) (width 0.25) (layer F.Cu) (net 18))
 (segment (start 69.6419 95.0771) (end 69.6419 114.6574) (width 0.25) (layer F.Cu) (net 18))
 (segment (start 69.6419 114.6574) (end 70.4275 115.443) (width 0.25) (layer F.Cu) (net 18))
 (segment (start 70.4275 115.443) (end 71.3353 115.443) (width 0.25) (layer F.Cu) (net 18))
 (segment (start 71.3353 115.443) (end 74.6091 118.7168) (width 0.25) (layer F.Cu) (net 18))
 (segment (start 74.6091 118.7168) (end 74.6091 121.1641) (width 0.25) (layer F.Cu) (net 18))
 (segment (start 74.6091 121.1641) (end 76.514 123.069) (width 0.25) (layer F.Cu) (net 18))
 (segment (start 76.514 123.069) (end 95.2277 123.069) (width 0.25) (layer F.Cu) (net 18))
 (segment (start 95.2277 123.069) (end 96.1302 122.1665) (width 0.25) (layer F.Cu) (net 18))
 (segment (start 96.1302 122.1665) (end 96.1302 121.285) (width 0.25) (layer F.Cu) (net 18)))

